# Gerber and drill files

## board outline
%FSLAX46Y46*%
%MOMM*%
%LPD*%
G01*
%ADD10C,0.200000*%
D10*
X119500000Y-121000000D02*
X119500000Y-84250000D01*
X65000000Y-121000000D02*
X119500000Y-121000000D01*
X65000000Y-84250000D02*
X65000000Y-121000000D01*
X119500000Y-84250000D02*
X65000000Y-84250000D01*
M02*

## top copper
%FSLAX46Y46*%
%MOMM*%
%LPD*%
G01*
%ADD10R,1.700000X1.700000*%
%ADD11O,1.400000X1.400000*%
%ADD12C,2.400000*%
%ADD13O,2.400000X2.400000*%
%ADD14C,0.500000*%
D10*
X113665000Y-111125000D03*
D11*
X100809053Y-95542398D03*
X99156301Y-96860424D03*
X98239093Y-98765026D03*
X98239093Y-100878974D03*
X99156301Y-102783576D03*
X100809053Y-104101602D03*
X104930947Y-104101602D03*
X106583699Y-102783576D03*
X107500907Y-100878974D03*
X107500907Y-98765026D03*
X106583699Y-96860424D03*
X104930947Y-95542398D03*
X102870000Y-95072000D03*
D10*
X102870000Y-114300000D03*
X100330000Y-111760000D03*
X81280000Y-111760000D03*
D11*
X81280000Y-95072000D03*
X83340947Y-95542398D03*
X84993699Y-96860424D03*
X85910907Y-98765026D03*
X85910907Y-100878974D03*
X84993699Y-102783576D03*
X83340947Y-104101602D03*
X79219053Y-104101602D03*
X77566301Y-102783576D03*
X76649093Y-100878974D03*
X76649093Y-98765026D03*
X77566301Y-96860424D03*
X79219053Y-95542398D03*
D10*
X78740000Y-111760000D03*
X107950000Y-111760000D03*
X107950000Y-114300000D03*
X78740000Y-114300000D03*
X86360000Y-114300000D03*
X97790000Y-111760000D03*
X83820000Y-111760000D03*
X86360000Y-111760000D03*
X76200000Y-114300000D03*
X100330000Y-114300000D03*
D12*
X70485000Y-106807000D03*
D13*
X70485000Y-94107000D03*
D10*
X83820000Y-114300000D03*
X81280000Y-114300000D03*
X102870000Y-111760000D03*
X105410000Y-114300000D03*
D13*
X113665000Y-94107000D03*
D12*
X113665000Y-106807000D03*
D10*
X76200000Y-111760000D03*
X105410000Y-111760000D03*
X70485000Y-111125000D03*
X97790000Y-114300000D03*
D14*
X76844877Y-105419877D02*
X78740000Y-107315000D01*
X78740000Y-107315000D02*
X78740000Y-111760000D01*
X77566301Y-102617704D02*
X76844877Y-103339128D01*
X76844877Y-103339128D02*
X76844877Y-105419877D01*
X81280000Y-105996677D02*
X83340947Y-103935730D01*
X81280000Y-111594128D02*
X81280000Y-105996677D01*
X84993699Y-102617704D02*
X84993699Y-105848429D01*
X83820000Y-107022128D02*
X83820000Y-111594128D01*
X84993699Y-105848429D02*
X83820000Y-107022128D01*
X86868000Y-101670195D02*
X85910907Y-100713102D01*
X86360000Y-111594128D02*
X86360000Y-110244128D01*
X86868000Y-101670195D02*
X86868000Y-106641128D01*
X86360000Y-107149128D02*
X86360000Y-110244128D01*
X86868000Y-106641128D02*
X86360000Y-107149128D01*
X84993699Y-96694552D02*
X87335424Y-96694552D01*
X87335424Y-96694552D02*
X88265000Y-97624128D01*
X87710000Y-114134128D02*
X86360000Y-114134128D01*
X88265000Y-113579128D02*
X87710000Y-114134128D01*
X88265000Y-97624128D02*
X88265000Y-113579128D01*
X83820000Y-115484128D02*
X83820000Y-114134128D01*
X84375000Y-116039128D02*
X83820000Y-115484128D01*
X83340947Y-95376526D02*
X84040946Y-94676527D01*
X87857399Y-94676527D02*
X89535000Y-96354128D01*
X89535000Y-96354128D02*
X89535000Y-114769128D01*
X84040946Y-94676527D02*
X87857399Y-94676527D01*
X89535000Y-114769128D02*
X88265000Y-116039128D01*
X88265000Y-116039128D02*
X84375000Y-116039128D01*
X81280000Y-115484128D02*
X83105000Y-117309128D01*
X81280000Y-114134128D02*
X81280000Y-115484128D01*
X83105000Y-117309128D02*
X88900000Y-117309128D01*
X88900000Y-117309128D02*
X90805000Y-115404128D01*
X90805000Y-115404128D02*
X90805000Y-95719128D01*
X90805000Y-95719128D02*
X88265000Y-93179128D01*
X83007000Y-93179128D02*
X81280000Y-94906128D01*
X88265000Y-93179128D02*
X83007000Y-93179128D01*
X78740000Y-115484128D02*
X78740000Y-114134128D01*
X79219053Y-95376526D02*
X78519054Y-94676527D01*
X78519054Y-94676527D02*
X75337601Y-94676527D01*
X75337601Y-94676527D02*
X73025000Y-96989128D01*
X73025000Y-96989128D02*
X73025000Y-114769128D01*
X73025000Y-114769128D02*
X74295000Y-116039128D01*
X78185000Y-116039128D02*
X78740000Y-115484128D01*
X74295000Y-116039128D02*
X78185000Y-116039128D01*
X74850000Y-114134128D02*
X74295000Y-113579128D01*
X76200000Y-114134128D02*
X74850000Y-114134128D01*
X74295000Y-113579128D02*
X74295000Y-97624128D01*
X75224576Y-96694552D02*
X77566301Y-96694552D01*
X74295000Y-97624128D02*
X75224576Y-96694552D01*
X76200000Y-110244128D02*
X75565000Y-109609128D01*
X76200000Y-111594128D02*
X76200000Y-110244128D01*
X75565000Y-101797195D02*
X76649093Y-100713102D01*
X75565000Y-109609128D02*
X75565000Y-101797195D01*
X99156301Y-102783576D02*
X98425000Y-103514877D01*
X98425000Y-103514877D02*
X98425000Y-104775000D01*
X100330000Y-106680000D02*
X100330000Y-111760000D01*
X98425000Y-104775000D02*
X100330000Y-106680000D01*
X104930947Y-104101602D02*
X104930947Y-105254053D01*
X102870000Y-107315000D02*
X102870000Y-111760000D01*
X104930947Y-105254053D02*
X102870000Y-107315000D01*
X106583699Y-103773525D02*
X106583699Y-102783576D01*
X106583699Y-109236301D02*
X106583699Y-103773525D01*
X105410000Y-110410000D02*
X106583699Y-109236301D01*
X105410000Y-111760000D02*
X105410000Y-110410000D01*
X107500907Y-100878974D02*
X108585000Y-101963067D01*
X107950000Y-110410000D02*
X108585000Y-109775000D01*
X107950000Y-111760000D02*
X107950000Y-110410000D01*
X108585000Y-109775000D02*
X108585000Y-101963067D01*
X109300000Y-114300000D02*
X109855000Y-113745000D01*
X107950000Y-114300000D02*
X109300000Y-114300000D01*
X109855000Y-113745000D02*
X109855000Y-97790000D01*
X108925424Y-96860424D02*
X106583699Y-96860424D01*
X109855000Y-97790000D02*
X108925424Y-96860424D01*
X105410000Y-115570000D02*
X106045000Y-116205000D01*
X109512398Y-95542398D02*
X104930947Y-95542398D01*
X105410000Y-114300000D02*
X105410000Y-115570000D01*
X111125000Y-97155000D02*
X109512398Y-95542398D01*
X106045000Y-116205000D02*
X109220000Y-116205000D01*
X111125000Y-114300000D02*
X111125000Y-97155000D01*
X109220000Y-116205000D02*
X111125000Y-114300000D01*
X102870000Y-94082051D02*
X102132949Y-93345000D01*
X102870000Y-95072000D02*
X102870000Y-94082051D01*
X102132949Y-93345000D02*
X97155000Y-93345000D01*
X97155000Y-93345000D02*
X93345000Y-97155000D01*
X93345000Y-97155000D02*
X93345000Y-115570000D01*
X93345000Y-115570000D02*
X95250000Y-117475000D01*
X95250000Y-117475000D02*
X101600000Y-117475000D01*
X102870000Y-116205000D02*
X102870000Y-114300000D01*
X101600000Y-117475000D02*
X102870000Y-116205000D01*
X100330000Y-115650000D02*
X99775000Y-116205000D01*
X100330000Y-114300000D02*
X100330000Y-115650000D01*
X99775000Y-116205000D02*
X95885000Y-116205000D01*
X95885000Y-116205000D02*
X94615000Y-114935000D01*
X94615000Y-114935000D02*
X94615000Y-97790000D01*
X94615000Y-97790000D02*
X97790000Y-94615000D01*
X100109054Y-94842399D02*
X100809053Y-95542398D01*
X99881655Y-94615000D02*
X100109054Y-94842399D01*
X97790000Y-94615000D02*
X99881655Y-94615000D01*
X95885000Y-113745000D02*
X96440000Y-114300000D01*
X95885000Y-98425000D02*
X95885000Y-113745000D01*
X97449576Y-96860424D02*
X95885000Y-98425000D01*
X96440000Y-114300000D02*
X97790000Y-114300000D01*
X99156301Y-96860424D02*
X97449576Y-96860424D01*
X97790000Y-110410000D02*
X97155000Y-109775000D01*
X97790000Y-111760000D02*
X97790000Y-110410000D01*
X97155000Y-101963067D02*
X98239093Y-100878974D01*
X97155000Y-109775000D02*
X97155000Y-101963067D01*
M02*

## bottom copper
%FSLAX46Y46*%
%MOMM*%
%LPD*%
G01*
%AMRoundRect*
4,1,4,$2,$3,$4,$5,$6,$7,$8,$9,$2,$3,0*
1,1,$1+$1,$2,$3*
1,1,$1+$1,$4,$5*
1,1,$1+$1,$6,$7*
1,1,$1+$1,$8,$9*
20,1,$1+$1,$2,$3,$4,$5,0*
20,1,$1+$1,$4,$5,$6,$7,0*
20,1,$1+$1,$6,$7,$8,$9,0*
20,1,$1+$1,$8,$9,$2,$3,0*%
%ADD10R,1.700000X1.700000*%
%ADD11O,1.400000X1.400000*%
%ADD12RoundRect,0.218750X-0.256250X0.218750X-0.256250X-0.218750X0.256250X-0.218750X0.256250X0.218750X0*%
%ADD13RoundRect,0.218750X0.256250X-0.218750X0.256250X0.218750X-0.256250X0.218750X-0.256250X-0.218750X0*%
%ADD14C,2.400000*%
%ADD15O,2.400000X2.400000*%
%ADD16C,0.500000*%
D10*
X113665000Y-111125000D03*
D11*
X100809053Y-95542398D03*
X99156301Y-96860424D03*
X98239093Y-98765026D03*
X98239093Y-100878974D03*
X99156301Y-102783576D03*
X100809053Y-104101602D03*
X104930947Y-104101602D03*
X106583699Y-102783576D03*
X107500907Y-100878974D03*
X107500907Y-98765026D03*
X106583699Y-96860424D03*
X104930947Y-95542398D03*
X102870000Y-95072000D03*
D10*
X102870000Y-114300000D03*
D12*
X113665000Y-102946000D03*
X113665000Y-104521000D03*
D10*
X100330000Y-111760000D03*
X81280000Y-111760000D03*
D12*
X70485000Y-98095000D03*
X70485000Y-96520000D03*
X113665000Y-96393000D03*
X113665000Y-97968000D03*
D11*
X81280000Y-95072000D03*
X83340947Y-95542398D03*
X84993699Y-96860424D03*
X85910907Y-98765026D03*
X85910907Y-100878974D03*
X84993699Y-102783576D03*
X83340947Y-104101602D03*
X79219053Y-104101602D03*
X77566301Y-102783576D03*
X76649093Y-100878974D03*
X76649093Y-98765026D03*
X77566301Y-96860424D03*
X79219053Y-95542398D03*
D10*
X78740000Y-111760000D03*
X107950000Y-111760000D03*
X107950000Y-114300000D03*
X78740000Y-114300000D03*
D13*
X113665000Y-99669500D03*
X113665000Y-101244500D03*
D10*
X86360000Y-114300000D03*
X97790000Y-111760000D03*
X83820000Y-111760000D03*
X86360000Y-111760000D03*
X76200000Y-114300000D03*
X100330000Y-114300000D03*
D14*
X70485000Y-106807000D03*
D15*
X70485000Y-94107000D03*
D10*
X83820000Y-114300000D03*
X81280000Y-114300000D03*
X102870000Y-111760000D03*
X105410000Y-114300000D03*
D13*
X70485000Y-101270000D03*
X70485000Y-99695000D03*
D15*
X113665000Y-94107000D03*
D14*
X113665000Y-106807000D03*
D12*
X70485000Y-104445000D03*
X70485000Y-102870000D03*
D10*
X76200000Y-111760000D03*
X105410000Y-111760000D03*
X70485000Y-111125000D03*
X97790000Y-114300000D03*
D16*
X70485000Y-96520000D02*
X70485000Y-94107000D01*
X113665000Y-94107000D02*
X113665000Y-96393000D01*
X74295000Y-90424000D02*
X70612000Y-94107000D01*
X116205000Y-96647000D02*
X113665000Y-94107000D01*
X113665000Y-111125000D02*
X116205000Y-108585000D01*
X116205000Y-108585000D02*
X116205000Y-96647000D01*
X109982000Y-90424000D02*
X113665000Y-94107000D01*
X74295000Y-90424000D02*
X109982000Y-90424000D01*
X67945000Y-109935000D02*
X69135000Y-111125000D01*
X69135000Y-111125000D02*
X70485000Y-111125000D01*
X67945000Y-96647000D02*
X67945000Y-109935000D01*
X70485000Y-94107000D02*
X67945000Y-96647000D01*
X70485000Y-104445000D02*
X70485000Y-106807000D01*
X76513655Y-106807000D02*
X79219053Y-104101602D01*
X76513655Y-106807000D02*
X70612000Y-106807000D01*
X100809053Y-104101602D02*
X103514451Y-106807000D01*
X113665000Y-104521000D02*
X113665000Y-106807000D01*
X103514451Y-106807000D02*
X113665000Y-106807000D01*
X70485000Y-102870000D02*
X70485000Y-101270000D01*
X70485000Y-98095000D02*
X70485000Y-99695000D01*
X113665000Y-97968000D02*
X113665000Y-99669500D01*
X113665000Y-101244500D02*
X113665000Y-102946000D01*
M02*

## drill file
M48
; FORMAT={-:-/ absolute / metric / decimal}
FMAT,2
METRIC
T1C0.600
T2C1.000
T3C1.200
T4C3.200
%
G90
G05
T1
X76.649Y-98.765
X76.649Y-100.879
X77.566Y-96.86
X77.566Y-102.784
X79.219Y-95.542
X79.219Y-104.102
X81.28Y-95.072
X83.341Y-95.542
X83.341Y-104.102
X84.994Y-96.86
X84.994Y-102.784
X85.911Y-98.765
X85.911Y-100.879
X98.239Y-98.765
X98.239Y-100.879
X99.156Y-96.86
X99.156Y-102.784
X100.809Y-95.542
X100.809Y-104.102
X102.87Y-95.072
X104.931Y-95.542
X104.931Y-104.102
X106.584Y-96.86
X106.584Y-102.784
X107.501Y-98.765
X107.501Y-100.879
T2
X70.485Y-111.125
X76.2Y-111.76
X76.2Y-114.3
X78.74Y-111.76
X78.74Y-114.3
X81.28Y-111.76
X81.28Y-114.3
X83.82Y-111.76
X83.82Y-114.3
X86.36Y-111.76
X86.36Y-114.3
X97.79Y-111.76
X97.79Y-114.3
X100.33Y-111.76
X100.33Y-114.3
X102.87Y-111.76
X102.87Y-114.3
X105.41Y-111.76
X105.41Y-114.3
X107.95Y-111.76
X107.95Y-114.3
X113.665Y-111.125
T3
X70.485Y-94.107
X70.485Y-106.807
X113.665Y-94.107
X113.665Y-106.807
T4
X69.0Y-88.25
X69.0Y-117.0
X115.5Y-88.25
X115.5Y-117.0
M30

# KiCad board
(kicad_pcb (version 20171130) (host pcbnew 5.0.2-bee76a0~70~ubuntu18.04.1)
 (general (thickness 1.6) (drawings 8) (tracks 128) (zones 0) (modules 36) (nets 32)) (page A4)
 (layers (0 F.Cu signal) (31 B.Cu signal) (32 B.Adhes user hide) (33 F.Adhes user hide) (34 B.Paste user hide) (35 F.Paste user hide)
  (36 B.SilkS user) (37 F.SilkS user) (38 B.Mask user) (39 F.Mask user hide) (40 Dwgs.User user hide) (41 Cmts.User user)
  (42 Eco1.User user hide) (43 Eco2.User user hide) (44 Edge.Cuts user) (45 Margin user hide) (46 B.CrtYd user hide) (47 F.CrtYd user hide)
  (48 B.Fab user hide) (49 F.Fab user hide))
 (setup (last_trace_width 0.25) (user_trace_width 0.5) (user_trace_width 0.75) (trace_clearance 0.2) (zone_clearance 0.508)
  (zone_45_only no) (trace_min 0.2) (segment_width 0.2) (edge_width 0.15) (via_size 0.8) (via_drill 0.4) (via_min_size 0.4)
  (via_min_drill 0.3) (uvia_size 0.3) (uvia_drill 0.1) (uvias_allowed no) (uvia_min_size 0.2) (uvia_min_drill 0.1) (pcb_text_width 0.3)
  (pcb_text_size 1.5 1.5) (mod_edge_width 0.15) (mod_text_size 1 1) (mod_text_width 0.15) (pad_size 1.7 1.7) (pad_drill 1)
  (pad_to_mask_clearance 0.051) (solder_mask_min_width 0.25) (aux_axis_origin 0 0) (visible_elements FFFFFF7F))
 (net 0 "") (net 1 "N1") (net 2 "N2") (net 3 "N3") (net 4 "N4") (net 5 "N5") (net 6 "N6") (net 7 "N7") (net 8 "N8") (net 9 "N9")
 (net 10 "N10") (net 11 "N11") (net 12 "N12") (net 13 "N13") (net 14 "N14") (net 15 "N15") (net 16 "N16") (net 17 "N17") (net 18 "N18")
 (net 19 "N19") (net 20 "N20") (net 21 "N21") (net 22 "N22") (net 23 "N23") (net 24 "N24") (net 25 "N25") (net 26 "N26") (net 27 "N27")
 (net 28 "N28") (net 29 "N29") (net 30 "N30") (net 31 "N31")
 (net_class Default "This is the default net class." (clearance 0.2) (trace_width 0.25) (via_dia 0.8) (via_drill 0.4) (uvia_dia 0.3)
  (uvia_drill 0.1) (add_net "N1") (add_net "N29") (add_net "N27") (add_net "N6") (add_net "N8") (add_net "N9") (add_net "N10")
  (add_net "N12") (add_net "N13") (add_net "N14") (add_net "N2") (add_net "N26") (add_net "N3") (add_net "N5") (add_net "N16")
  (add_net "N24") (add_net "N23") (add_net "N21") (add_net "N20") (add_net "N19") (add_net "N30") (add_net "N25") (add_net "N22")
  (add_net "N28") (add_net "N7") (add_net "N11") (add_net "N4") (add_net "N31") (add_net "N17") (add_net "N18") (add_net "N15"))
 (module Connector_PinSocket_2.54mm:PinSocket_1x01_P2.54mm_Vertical (layer F.Cu) (at 113.665 111.125)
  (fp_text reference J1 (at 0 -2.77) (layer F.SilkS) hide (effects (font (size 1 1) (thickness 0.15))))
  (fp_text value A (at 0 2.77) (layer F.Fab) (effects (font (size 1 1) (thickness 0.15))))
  (pad 1 thru_hole rect (at 0 0) (size 1.7 1.7) (drill 1) (layers *.Cu *.Mask) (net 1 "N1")))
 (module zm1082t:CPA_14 (layer F.Cu) (at 102.87 99.822)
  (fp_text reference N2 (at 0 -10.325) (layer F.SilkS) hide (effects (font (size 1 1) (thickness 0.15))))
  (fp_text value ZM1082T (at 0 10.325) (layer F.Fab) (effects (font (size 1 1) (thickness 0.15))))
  (pad 6 thru_hole oval (at -2.060947 -4.279602) (size 1.4 1.4) (drill 0.6) (layers *.Cu *.Mask) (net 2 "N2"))
  (pad 5 thru_hole oval (at -3.713699 -2.961576) (size 1.4 1.4) (drill 0.6) (layers *.Cu *.Mask) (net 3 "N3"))
  (pad 4 thru_hole oval (at -4.630907 -1.056974) (size 1.4 1.4) (drill 0.6) (layers *.Cu *.Mask) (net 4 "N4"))
  (pad 3 thru_hole oval (at -4.630907 1.056974) (size 1.4 1.4) (drill 0.6) (layers *.Cu *.Mask) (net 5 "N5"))
  (pad 2 thru_hole oval (at -3.713699 2.961576) (size 1.4 1.4) (drill 0.6) (layers *.Cu *.Mask) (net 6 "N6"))
  (pad 1 thru_hole oval (at -2.060947 4.279602) (size 1.4 1.4) (drill 0.6) (layers *.Cu *.Mask) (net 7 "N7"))
  (pad 13 thru_hole oval (at 2.060947 4.279602) (size 1.4 1.4) (drill 0.6) (layers *.Cu *.Mask) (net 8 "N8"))
  (pad 12 thru_hole oval (at 3.713699 2.961576) (size 1.4 1.4) (drill 0.6) (layers *.Cu *.Mask) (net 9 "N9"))
  (pad 11 thru_hole oval (at 4.630907 1.056974) (size 1.4 1.4) (drill 0.6) (layers *.Cu *.Mask) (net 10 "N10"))
  (pad 10 thru_hole oval (at 4.630907 -1.056974) (size 1.4 1.4) (drill 0.6) (layers *.Cu *.Mask) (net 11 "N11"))
  (pad 9 thru_hole oval (at 3.713699 -2.961576) (size 1.4 1.4) (drill 0.6) (layers *.Cu *.Mask) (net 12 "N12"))
  (pad 8 thru_hole oval (at 2.060947 -4.279602) (size 1.4 1.4) (drill 0.6) (layers *.Cu *.Mask) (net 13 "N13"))
  (pad 7 thru_hole oval (at 0 -4.75) (size 1.4 1.4) (drill 0.6) (layers *.Cu *.Mask) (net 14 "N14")))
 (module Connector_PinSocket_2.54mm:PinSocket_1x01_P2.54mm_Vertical (layer F.Cu) (at 102.87 114.3)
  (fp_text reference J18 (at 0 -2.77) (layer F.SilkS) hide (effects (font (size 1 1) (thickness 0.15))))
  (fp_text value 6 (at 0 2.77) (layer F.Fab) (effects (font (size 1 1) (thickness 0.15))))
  (pad 1 thru_hole rect (at 0 0) (size 1.7 1.7) (drill 1) (layers *.Cu *.Mask) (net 14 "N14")))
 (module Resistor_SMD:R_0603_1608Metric (layer B.Cu) (at 113.665 103.7335 270)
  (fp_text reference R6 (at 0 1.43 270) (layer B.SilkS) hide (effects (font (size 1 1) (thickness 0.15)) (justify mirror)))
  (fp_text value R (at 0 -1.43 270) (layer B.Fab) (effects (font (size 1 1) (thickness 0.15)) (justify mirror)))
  (pad 1 smd roundrect (at -0.7875 0 270) (size 0.875 0.95) (layers B.Cu B.Paste B.Mask) (roundrect_rratio 0.25) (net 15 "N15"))
  (pad 2 smd roundrect (at 0.7875 0 270) (size 0.875 0.95) (layers B.Cu B.Paste B.Mask) (roundrect_rratio 0.25) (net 7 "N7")))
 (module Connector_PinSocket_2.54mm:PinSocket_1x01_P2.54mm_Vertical (layer F.Cu) (at 100.33 111.76)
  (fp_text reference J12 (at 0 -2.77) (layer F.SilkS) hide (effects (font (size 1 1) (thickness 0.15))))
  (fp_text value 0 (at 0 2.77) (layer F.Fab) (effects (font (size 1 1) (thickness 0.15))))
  (pad 1 thru_hole rect (at 0 0) (size 1.7 1.7) (drill 1) (layers *.Cu *.Mask) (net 6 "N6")))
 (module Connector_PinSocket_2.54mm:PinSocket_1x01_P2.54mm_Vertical (layer F.Cu) (at 81.28 111.76)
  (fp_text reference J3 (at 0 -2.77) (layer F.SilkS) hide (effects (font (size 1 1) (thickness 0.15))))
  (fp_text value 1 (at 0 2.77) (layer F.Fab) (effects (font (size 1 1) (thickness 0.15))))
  (pad 1 thru_hole rect (at 0 0) (size 1.7 1.7) (drill 1) (layers *.Cu *.Mask) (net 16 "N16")))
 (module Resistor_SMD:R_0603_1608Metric (layer B.Cu) (at 70.485 97.3075 270)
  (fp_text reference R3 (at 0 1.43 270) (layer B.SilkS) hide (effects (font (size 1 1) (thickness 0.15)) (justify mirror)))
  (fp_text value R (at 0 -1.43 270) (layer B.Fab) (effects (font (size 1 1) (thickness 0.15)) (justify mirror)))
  (pad 2 smd roundrect (at 0.7875 0 270) (size 0.875 0.95) (layers B.Cu B.Paste B.Mask) (roundrect_rratio 0.25) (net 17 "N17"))
  (pad 1 smd roundrect (at -0.7875 0 270) (size 0.875 0.95) (layers B.Cu B.Paste B.Mask) (roundrect_rratio 0.25) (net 1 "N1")))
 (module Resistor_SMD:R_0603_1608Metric (layer B.Cu) (at 113.665 97.1805 270)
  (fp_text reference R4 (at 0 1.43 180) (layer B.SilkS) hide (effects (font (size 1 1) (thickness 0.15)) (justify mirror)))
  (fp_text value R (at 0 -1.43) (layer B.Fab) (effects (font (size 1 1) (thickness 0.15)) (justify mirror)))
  (pad 1 smd roundrect (at -0.7875 0 270) (size 0.875 0.95) (layers B.Cu B.Paste B.Mask) (roundrect_rratio 0.25) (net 1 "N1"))
  (pad 2 smd roundrect (at 0.7875 0 270) (size 0.875 0.95) (layers B.Cu B.Paste B.Mask) (roundrect_rratio 0.25) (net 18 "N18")))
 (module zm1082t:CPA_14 (layer F.Cu) (at 81.28 99.822)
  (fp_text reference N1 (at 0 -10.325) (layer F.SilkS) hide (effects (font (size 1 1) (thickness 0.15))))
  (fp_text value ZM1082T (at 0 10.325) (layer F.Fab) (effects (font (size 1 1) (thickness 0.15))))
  (pad 7 thru_hole oval (at 0 -4.75) (size 1.4 1.4) (drill 0.6) (layers *.Cu *.Mask) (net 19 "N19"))
  (pad 8 thru_hole oval (at 2.060947 -4.279602) (size 1.4 1.4) (drill 0.6) (layers *.Cu *.Mask) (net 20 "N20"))
  (pad 9 thru_hole oval (at 3.713699 -2.961576) (size 1.4 1.4) (drill 0.6) (layers *.Cu *.Mask) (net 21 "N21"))
  (pad 10 thru_hole oval (at 4.630907 -1.056974) (size 1.4 1.4) (drill 0.6) (layers *.Cu *.Mask) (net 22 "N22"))
  (pad 11 thru_hole oval (at 4.630907 1.056974) (size 1.4 1.4) (drill 0.6) (layers *.Cu *.Mask) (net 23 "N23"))
  (pad 12 thru_hole oval (at 3.713699 2.961576) (size 1.4 1.4) (drill 0.6) (layers *.Cu *.Mask) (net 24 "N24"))
  (pad 13 thru_hole oval (at 2.060947 4.279602) (size 1.4 1.4) (drill 0.6) (layers *.Cu *.Mask) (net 16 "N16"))
  (pad 1 thru_hole oval (at -2.060947 4.279602) (size 1.4 1.4) (drill 0.6) (layers *.Cu *.Mask) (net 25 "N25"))
  (pad 2 thru_hole oval (at -3.713699 2.961576) (size 1.4 1.4) (drill 0.6) (layers *.Cu *.Mask) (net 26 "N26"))
  (pad 3 thru_hole oval (at -4.630907 1.056974) (size 1.4 1.4) (drill 0.6) (layers *.Cu *.Mask) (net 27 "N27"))
  (pad 4 thru_hole oval (at -4.630907 -1.056974) (size 1.4 1.4) (drill 0.6) (layers *.Cu *.Mask) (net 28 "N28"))
  (pad 5 thru_hole oval (at -3.713699 -2.961576) (size 1.4 1.4) (drill 0.6) (layers *.Cu *.Mask) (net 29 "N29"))
  (pad 6 thru_hole oval (at -2.060947 -4.279602) (size 1.4 1.4) (drill 0.6) (layers *.Cu *.Mask) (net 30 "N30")))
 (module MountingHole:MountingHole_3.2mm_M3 (layer F.Cu) (at 69 88.25)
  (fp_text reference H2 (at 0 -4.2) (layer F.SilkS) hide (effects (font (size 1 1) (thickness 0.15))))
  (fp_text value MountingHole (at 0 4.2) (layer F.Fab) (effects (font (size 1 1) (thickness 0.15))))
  (pad 1 np_thru_hole circle (at 0 0) (size 3.2 3.2) (drill 3.2) (layers *.Cu *.Mask)))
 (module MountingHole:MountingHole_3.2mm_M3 (layer F.Cu) (at 115.5 117)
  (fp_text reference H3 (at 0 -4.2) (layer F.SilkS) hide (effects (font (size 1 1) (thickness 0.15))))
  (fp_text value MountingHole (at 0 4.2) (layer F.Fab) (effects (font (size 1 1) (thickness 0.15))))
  (pad 1 np_thru_hole circle (at 0 0) (size 3.2 3.2) (drill 3.2) (layers *.Cu *.Mask)))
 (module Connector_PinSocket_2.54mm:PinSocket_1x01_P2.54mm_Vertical (layer F.Cu) (at 78.74 113.03)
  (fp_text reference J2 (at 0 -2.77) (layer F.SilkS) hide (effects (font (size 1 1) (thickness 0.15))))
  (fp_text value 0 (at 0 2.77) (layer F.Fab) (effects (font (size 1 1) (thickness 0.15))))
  (pad 1 thru_hole rect (at 0 -1.27) (size 1.7 1.7) (drill 1) (layers *.Cu *.Mask) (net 26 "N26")))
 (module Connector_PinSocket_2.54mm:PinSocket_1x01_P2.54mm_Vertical (layer F.Cu) (at 107.95 111.76)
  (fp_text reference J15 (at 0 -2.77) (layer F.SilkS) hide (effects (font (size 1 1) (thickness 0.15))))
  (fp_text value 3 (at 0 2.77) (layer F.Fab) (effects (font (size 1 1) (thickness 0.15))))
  (pad 1 thru_hole rect (at 0 0) (size 1.7 1.7) (drill 1) (layers *.Cu *.Mask) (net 10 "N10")))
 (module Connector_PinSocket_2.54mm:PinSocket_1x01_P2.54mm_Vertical (layer F.Cu) (at 107.95 114.3)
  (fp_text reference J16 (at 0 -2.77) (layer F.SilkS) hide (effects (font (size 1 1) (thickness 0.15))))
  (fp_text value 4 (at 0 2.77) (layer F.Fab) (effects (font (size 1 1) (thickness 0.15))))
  (pad 1 thru_hole rect (at 0 0) (size 1.7 1.7) (drill 1) (layers *.Cu *.Mask) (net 12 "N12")))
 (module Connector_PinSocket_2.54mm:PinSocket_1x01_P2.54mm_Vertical (layer F.Cu) (at 78.74 114.3)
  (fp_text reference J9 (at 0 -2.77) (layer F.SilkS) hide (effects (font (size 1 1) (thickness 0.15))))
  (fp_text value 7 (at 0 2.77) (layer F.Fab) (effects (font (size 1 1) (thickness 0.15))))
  (pad 1 thru_hole rect (at 0 0) (size 1.7 1.7) (drill 1) (layers *.Cu *.Mask) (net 30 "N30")))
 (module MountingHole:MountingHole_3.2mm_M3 (layer F.Cu) (at 69 117)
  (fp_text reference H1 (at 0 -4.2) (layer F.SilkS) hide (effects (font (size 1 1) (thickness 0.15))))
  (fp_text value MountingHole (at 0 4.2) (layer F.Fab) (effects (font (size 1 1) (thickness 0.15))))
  (pad 1 np_thru_hole circle (at 0 0) (size 3.2 3.2) (drill 3.2) (layers *.Cu *.Mask)))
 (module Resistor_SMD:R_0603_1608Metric (layer B.Cu) (at 113.665 100.457 90)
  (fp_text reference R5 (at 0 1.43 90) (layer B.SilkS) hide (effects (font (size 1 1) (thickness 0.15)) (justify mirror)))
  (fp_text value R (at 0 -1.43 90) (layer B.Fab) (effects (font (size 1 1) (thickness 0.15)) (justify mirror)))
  (pad 2 smd roundrect (at 0.7875 0 90) (size 0.875 0.95) (layers B.Cu B.Paste B.Mask) (roundrect_rratio 0.25) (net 18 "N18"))
  (pad 1 smd roundrect (at -0.7875 0 90) (size 0.875 0.95) (layers B.Cu B.Paste B.Mask) (roundrect_rratio 0.25) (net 15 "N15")))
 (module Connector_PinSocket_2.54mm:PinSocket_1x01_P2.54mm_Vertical (layer F.Cu) (at 86.36 114.3)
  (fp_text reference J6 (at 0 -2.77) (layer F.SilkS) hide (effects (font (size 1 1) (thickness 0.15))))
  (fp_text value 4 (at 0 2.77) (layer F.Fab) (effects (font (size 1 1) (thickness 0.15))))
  (pad 1 thru_hole rect (at 0 0) (size 1.7 1.7) (drill 1) (layers *.Cu *.Mask) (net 21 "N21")))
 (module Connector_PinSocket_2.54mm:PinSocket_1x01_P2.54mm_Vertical (layer F.Cu) (at 97.79 111.76)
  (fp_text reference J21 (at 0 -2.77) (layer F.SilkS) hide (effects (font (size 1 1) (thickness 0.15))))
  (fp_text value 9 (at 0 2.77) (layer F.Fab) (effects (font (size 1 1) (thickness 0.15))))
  (pad 1 thru_hole rect (at 0 0) (size 1.7 1.7) (drill 1) (layers *.Cu *.Mask) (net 5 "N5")))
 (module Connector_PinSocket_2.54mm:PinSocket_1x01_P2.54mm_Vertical (layer F.Cu) (at 83.82 111.76)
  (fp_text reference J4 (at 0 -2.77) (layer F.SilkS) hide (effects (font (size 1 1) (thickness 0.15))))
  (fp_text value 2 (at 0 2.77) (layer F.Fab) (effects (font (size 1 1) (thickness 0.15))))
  (pad 1 thru_hole rect (at 0 0) (size 1.7 1.7) (drill 1) (layers *.Cu *.Mask) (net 24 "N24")))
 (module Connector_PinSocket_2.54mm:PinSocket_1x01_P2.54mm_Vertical (layer F.Cu) (at 86.36 111.76)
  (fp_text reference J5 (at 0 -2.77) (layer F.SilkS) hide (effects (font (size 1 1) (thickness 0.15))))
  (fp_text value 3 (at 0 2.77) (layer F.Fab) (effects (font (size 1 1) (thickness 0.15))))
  (pad 1 thru_hole rect (at 0 0) (size 1.7 1.7) (drill 1) (layers *.Cu *.Mask) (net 23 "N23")))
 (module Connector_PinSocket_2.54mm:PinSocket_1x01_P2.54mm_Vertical (layer F.Cu) (at 76.2 114.3)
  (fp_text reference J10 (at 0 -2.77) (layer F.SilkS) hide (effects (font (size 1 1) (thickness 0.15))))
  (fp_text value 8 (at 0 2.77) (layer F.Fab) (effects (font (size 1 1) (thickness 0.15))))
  (pad 1 thru_hole rect (at 0 0) (size 1.7 1.7) (drill 1) (layers *.Cu *.Mask) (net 29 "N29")))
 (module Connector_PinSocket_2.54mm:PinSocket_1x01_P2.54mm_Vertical (layer F.Cu) (at 100.33 114.3)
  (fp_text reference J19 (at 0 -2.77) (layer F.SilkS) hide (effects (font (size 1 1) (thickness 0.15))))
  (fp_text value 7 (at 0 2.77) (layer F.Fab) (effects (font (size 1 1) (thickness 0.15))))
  (pad 1 thru_hole rect (at 0 0) (size 1.7 1.7) (drill 1) (layers *.Cu *.Mask) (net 2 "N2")))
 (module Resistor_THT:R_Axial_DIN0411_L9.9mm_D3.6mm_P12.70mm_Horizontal (layer B.Cu) (at 70.485 106.807 90)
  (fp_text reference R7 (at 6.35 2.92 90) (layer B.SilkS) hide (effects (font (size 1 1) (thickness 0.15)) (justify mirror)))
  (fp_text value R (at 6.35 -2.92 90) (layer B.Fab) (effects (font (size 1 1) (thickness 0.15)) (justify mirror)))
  (pad 1 thru_hole circle (at 0 0 90) (size 2.4 2.4) (drill 1.2) (layers *.Cu *.Mask) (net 25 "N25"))
  (pad 2 thru_hole oval (at 12.7 0 90) (size 2.4 2.4) (drill 1.2) (layers *.Cu *.Mask) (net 1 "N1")))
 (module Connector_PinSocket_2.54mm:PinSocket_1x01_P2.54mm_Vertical (layer F.Cu) (at 83.82 114.3)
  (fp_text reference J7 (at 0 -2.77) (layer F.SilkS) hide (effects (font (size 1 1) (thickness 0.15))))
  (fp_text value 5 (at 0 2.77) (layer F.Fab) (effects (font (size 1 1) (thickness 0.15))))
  (pad 1 thru_hole rect (at 0 0) (size 1.7 1.7) (drill 1) (layers *.Cu *.Mask) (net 20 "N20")))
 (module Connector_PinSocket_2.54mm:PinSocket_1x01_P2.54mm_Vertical (layer F.Cu) (at 81.28 114.3)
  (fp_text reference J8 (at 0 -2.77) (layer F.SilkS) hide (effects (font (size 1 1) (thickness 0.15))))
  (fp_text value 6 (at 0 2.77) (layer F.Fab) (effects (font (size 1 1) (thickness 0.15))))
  (pad 1 thru_hole rect (at 0 0) (size 1.7 1.7) (drill 1) (layers *.Cu *.Mask) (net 19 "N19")))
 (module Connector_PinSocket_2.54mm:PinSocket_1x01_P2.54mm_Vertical (layer F.Cu) (at 102.87 111.76)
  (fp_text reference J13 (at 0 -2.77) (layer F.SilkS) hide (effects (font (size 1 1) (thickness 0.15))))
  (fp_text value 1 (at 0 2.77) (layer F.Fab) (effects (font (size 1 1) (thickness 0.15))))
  (pad 1 thru_hole rect (at 0 0) (size 1.7 1.7) (drill 1) (layers *.Cu *.Mask) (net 8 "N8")))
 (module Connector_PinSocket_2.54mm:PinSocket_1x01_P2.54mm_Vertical (layer F.Cu) (at 105.41 114.3)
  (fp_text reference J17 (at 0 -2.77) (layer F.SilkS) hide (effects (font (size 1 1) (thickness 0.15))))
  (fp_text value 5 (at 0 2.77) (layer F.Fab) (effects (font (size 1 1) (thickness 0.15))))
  (pad 1 thru_hole rect (at 0 0) (size 1.7 1.7) (drill 1) (layers *.Cu *.Mask) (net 13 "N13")))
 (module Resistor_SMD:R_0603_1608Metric (layer B.Cu) (at 70.485 100.4825 90)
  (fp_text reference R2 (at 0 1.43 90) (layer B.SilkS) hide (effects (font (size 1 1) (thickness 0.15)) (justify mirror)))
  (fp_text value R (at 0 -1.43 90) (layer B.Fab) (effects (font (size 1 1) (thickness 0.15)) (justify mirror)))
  (pad 1 smd roundrect (at -0.7875 0 90) (size 0.875 0.95) (layers B.Cu B.Paste B.Mask) (roundrect_rratio 0.25) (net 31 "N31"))
  (pad 2 smd roundrect (at 0.7875 0 90) (size 0.875 0.95) (layers B.Cu B.Paste B.Mask) (roundrect_rratio 0.25) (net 17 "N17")))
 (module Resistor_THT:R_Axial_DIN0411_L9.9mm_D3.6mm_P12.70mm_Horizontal (layer B.Cu) (at 113.665 106.807 90)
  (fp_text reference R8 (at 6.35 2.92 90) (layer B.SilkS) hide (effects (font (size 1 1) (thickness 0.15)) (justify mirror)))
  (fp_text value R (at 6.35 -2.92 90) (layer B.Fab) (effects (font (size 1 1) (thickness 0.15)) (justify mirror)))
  (pad 2 thru_hole oval (at 12.7 0 90) (size 2.4 2.4) (drill 1.2) (layers *.Cu *.Mask) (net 1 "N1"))
  (pad 1 thru_hole circle (at 0 0 90) (size 2.4 2.4) (drill 1.2) (layers *.Cu *.Mask) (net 7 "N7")))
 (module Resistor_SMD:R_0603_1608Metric (layer B.Cu) (at 70.485 103.6575 270)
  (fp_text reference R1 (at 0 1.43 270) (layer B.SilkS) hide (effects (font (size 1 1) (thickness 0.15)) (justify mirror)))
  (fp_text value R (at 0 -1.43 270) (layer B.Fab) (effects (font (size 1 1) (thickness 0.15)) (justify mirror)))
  (pad 2 smd roundrect (at 0.7875 0 270) (size 0.875 0.95) (layers B.Cu B.Paste B.Mask) (roundrect_rratio 0.25) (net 25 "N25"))
  (pad 1 smd roundrect (at -0.7875 0 270) (size 0.875 0.95) (layers B.Cu B.Paste B.Mask) (roundrect_rratio 0.25) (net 31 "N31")))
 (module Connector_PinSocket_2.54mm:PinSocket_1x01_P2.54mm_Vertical (layer F.Cu) (at 76.2 111.76)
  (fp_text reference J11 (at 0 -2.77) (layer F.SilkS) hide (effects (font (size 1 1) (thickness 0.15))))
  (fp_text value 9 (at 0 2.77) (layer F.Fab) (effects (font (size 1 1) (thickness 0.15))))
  (pad 1 thru_hole rect (at 0 0) (size 1.7 1.7) (drill 1) (layers *.Cu *.Mask) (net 27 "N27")))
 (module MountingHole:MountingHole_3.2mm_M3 (layer F.Cu) (at 115.5 88.25)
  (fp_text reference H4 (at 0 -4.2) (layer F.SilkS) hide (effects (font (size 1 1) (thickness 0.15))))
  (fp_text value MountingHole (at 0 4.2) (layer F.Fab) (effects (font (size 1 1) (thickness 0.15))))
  (pad 1 np_thru_hole circle (at 0 0) (size 3.2 3.2) (drill 3.2) (layers *.Cu *.Mask)))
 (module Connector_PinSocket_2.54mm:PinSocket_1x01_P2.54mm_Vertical (layer F.Cu) (at 105.41 111.76)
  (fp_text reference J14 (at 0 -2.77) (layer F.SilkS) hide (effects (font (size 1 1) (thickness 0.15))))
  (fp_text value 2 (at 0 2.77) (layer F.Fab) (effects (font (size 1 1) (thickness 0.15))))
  (pad 1 thru_hole rect (at 0 0) (size 1.7 1.7) (drill 1) (layers *.Cu *.Mask) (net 9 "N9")))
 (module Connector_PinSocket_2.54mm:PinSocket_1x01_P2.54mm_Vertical (layer F.Cu) (at 70.485 111.125)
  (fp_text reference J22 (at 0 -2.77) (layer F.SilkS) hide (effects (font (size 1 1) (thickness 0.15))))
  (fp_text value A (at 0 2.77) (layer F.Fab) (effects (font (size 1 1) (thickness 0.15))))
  (pad 1 thru_hole rect (at 0 0) (size 1.7 1.7) (drill 1) (layers *.Cu *.Mask) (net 1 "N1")))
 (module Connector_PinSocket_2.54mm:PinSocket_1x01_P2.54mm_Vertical (layer F.Cu) (at 97.79 114.3)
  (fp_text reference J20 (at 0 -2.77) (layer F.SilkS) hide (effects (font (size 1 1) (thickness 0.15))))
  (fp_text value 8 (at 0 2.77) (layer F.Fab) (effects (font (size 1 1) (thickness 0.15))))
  (pad 1 thru_hole rect (at 0 0) (size 1.7 1.7) (drill 1) (layers *.Cu *.Mask) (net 3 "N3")))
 (gr_line (start 119.5 121) (end 119.5 84.25) (layer Edge.Cuts) (width 0.2))
 (gr_line (start 65 121) (end 119.5 121) (layer Edge.Cuts) (width 0.2))
 (gr_line (start 65 84.25) (end 65 121) (layer Edge.Cuts) (width 0.2))
 (gr_line (start 119.5 84.25) (end 65 84.25) (layer Edge.Cuts) (width 0.2))
 (segment (start 70.485 96.52) (end 70.485 94.107) (width 0.5) (layer B.Cu) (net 1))
 (segment (start 113.665 94.107) (end 113.665 96.393) (width 0.5) (layer B.Cu) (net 1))
 (segment (start 74.295 90.424) (end 70.612 94.107) (width 0.5) (layer B.Cu) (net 1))
 (segment (start 116.205 96.647) (end 113.665 94.107) (width 0.5) (layer B.Cu) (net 1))
 (segment (start 113.665 111.125) (end 116.205 108.585) (width 0.5) (layer B.Cu) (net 1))
 (segment (start 116.205 108.585) (end 116.205 96.647) (width 0.5) (layer B.Cu) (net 1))
 (segment (start 109.982 90.424) (end 113.665 94.107) (width 0.5) (layer B.Cu) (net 1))
 (segment (start 74.295 90.424) (end 109.982 90.424) (width 0.5) (layer B.Cu) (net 1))
 (segment (start 67.945 109.935) (end 69.135 111.125) (width 0.5) (layer B.Cu) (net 1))
 (segment (start 69.135 111.125) (end 70.485 111.125) (width 0.5) (layer B.Cu) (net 1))
 (segment (start 67.945 96.647) (end 67.945 109.935) (width 0.5) (layer B.Cu) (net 1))
 (segment (start 70.485 94.107) (end 67.945 96.647) (width 0.5) (layer B.Cu) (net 1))
 (segment (start 76.844877 105.419877) (end 78.74 107.315) (width 0.5) (layer F.Cu) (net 26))
 (segment (start 78.74 107.315) (end 78.74 111.76) (width 0.5) (layer F.Cu) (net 26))
 (segment (start 77.566301 102.617704) (end 76.844877 103.339128) (width 0.5) (layer F.Cu) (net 26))
 (segment (start 76.844877 103.339128) (end 76.844877 105.419877) (width 0.5) (layer F.Cu) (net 26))
 (segment (start 81.28 105.996677) (end 83.340947 103.93573) (width 0.5) (layer F.Cu) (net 16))
 (segment (start 81.28 111.594128) (end 81.28 105.996677) (width 0.5) (layer F.Cu) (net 16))
 (segment (start 84.993699 102.617704) (end 84.993699 105.848429) (width 0.5) (layer F.Cu) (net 24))
 (segment (start 83.82 107.022128) (end 83.82 111.594128) (width 0.5) (layer F.Cu) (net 24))
 (segment (start 84.993699 105.848429) (end 83.82 107.022128) (width 0.5) (layer F.Cu) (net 24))
 (segment (start 86.868 101.670195) (end 85.910907 100.713102) (width 0.5) (layer F.Cu) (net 23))
 (segment (start 86.36 111.594128) (end 86.36 110.244128) (width 0.5) (layer F.Cu) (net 23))
 (segment (start 86.868 101.670195) (end 86.868 106.641128) (width 0.5) (layer F.Cu) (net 23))
 (segment (start 86.36 107.149128) (end 86.36 110.244128) (width 0.5) (layer F.Cu) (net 23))
 (segment (start 86.868 106.641128) (end 86.36 107.149128) (width 0.5) (layer F.Cu) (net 23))
 (segment (start 84.993699 96.694552) (end 87.335424 96.694552) (width 0.5) (layer F.Cu) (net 21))
 (segment (start 87.335424 96.694552) (end 88.265 97.624128) (width 0.5) (layer F.Cu) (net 21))
 (segment (start 87.71 114.134128) (end 86.36 114.134128) (width 0.5) (layer F.Cu) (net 21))
 (segment (start 88.265 113.579128) (end 87.71 114.134128) (width 0.5) (layer F.Cu) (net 21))
 (segment (start 88.265 97.624128) (end 88.265 113.579128) (width 0.5) (layer F.Cu) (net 21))
 (segment (start 83.82 115.484128) (end 83.82 114.134128) (width 0.5) (layer F.Cu) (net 20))
 (segment (start 84.375 116.039128) (end 83.82 115.484128) (width 0.5) (layer F.Cu) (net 20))
 (segment (start 83.340947 95.376526) (end 84.040946 94.676527) (width 0.5) (layer F.Cu) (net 20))
 (segment (start 87.857399 94.676527) (end 89.535 96.354128) (width 0.5) (layer F.Cu) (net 20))
 (segment (start 89.535 96.354128) (end 89.535 114.769128) (width 0.5) (layer F.Cu) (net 20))
 (segment (start 84.040946 94.676527) (end 87.857399 94.676527) (width 0.5) (layer F.Cu) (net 20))
 (segment (start 89.535 114.769128) (end 88.265 116.039128) (width 0.5) (layer F.Cu) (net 20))
 (segment (start 88.265 116.039128) (end 84.375 116.039128) (width 0.5) (layer F.Cu) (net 20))
 (segment (start 81.28 115.484128) (end 83.105 117.309128) (width 0.5) (layer F.Cu) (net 19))
 (segment (start 81.28 114.134128) (end 81.28 115.484128) (width 0.5) (layer F.Cu) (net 19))
 (segment (start 83.105 117.309128) (end 88.9 117.309128) (width 0.5) (layer F.Cu) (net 19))
 (segment (start 88.9 117.309128) (end 90.805 115.404128) (width 0.5) (layer F.Cu) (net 19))
 (segment (start 90.805 115.404128) (end 90.805 95.719128) (width 0.5) (layer F.Cu) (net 19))
 (segment (start 90.805 95.719128) (end 88.265 93.179128) (width 0.5) (layer F.Cu) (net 19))
 (segment (start 83.007 93.179128) (end 81.28 94.906128) (width 0.5) (layer F.Cu) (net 19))
 (segment (start 88.265 93.179128) (end 83.007 93.179128) (width 0.5) (layer F.Cu) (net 19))
 (segment (start 78.74 115.484128) (end 78.74 114.134128) (width 0.5) (layer F.Cu) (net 30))
 (segment (start 79.219053 95.376526) (end 78.519054 94.676527) (width 0.5) (layer F.Cu) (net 30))
 (segment (start 78.519054 94.676527) (end 75.337601 94.676527) (width 0.5) (layer F.Cu) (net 30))
 (segment (start 75.337601 94.676527) (end 73.025 96.989128) (width 0.5) (layer F.Cu) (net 30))
 (segment (start 73.025 96.989128) (end 73.025 114.769128) (width 0.5) (layer F.Cu) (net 30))
 (segment (start 73.025 114.769128) (end 74.295 116.039128) (width 0.5) (layer F.Cu) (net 30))
 (segment (start 78.185 116.039128) (end 78.74 115.484128) (width 0.5) (layer F.Cu) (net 30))
 (segment (start 74.295 116.039128) (end 78.185 116.039128) (width 0.5) (layer F.Cu) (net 30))
 (segment (start 74.85 114.134128) (end 74.295 113.579128) (width 0.5) (layer F.Cu) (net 29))
 (segment (start 76.2 114.134128) (end 74.85 114.134128) (width 0.5) (layer F.Cu) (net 29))
 (segment (start 74.295 113.579128) (end 74.295 97.624128) (width 0.5) (layer F.Cu) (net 29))
 (segment (start 75.224576 96.694552) (end 77.566301 96.694552) (width 0.5) (layer F.Cu) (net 29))
 (segment (start 74.295 97.624128) (end 75.224576 96.694552) (width 0.5) (layer F.Cu) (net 29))
 (segment (start 76.2 110.244128) (end 75.565 109.609128) (width 0.5) (layer F.Cu) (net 27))
 (segment (start 76.2 111.594128) (end 76.2 110.244128) (width 0.5) (layer F.Cu) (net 27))
 (segment (start 75.565 101.797195) (end 76.649093 100.713102) (width 0.5) (layer F.Cu) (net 27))
 (segment (start 75.565 109.609128) (end 75.565 101.797195) (width 0.5) (layer F.Cu) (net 27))
 (segment (start 99.156301 102.783576) (end 98.425 103.514877) (width 0.5) (layer F.Cu) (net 6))
 (segment (start 98.425 103.514877) (end 98.425 104.775) (width 0.5) (layer F.Cu) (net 6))
 (segment (start 100.33 106.68) (end 100.33 111.76) (width 0.5) (layer F.Cu) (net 6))
 (segment (start 98.425 104.775) (end 100.33 106.68) (width 0.5) (layer F.Cu) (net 6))
 (segment (start 104.930947 104.101602) (end 104.930947 105.254053) (width 0.5) (layer F.Cu) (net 8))
 (segment (start 102.87 107.315) (end 102.87 111.76) (width 0.5) (layer F.Cu) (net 8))
 (segment (start 104.930947 105.254053) (end 102.87 107.315) (width 0.5) (layer F.Cu) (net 8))
 (segment (start 106.583699 103.773525) (end 106.583699 102.783576) (width 0.5) (layer F.Cu) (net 9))
 (segment (start 106.583699 109.236301) (end 106.583699 103.773525) (width 0.5) (layer F.Cu) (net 9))
 (segment (start 105.41 110.41) (end 106.583699 109.236301) (width 0.5) (layer F.Cu) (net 9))
 (segment (start 105.41 111.76) (end 105.41 110.41) (width 0.5) (layer F.Cu) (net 9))
 (segment (start 107.500907 100.878974) (end 108.585 101.963067) (width 0.5) (layer F.Cu) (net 10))
 (segment (start 107.95 110.41) (end 108.585 109.775) (width 0.5) (layer F.Cu) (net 10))
 (segment (start 107.95 111.76) (end 107.95 110.41) (width 0.5) (layer F.Cu) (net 10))
 (segment (start 108.585 109.775) (end 108.585 101.963067) (width 0.5) (layer F.Cu) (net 10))
 (segment (start 109.3 114.3) (end 109.855 113.745) (width 0.5) (layer F.Cu) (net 12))
 (segment (start 107.95 114.3) (end 109.3 114.3) (width 0.5) (layer F.Cu) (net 12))
 (segment (start 109.855 113.745) (end 109.855 97.79) (width 0.5) (layer F.Cu) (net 12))
 (segment (start 108.925424 96.860424) (end 106.583699 96.860424) (width 0.5) (layer F.Cu) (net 12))
 (segment (start 109.855 97.79) (end 108.925424 96.860424) (width 0.5) (layer F.Cu) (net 12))
 (segment (start 105.41 115.57) (end 106.045 116.205) (width 0.5) (layer F.Cu) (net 13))
 (segment (start 109.512398 95.542398) (end 104.930947 95.542398) (width 0.5) (layer F.Cu) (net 13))
 (segment (start 105.41 114.3) (end 105.41 115.57) (width 0.5) (layer F.Cu) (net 13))
 (segment (start 111.125 97.155) (end 109.512398 95.542398) (width 0.5) (layer F.Cu) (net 13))
 (segment (start 106.045 116.205) (end 109.22 116.205) (width 0.5) (layer F.Cu) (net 13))
 (segment (start 111.125 114.3) (end 111.125 97.155) (width 0.5) (layer F.Cu) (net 13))
 (segment (start 109.22 116.205) (end 111.125 114.3) (width 0.5) (layer F.Cu) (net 13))
 (segment (start 102.87 94.082051) (end 102.132949 93.345) (width 0.5) (layer F.Cu) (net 14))
 (segment (start 102.87 95.072) (end 102.87 94.082051) (width 0.5) (layer F.Cu) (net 14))
 (segment (start 102.132949 93.345) (end 97.155 93.345) (width 0.5) (layer F.Cu) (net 14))
 (segment (start 97.155 93.345) (end 93.345 97.155) (width 0.5) (layer F.Cu) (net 14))
 (segment (start 93.345 97.155) (end 93.345 115.57) (width 0.5) (layer F.Cu) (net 14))
 (segment (start 93.345 115.57) (end 95.25 117.475) (width 0.5) (layer F.Cu) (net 14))
 (segment (start 95.25 117.475) (end 101.6 117.475) (width 0.5) (layer F.Cu) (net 14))
 (segment (start 102.87 116.205) (end 102.87 114.3) (width 0.5) (layer F.Cu) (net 14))
 (segment (start 101.6 117.475) (end 102.87 116.205) (width 0.5) (layer F.Cu) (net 14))
 (segment (start 100.33 115.65) (end 99.775 116.205) (width 0.5) (layer F.Cu) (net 2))
 (segment (start 100.33 114.3) (end 100.33 115.65) (width 0.5) (layer F.Cu) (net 2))
 (segment (start 99.775 116.205) (end 95.885 116.205) (width 0.5) (layer F.Cu) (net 2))
 (segment (start 95.885 116.205) (end 94.615 114.935) (width 0.5) (layer F.Cu) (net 2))
 (segment (start 94.615 114.935) (end 94.615 97.79) (width 0.5) (layer F.Cu) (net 2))
 (segment (start 94.615 97.79) (end 97.79 94.615) (width 0.5) (layer F.Cu) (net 2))
 (segment (start 100.109054 94.842399) (end 100.809053 95.542398) (width 0.5) (layer F.Cu) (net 2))
 (segment (start 99.881655 94.615) (end 100.109054 94.842399) (width 0.5) (layer F.Cu) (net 2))
 (segment (start 97.79 94.615) (end 99.881655 94.615) (width 0.5) (layer F.Cu) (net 2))
 (segment (start 95.885 113.745) (end 96.44 114.3) (width 0.5) (layer F.Cu) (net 3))
 (segment (start 95.885 98.425) (end 95.885 113.745) (width 0.5) (layer F.Cu) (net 3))
 (segment (start 97.449576 96.860424) (end 95.885 98.425) (width 0.5) (layer F.Cu) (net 3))
 (segment (start 96.44 114.3) (end 97.79 114.3) (width 0.5) (layer F.Cu) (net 3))
 (segment (start 99.156301 96.860424) (end 97.449576 96.860424) (width 0.5) (layer F.Cu) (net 3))
 (segment (start 97.79 110.41) (end 97.155 109.775) (width 0.5) (layer F.Cu) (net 5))
 (segment (start 97.79 111.76) (end 97.79 110.41) (width 0.5) (layer F.Cu) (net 5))
 (segment (start 97.155 101.963067) (end 98.239093 100.878974) (width 0.5) (layer F.Cu) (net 5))
 (segment (start 97.155 109.775) (end 97.155 101.963067) (width 0.5) (layer F.Cu) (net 5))
 (segment (start 70.485 104.445) (end 70.485 106.807) (width 0.5) (layer B.Cu) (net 25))
 (segment (start 76.513655 106.807) (end 79.219053 104.101602) (width 0.5) (layer B.Cu) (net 25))
 (segment (start 76.513655 106.807) (end 70.612 106.807) (width 0.5) (layer B.Cu) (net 25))
 (segment (start 100.809053 104.101602) (end 103.514451 106.807) (width 0.5) (layer B.Cu) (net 7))
 (segment (start 113.665 104.521) (end 113.665 106.807) (width 0.5) (layer B.Cu) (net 7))
 (segment (start 103.514451 106.807) (end 113.665 106.807) (width 0.5) (layer B.Cu) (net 7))
 (segment (start 70.485 102.87) (end 70.485 101.27) (width 0.5) (layer B.Cu) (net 31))
 (segment (start 70.485 98.095) (end 70.485 99.695) (width 0.5) (layer B.Cu) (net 17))
 (segment (start 113.665 97.968) (end 113.665 99.6695) (width 0.5) (layer B.Cu) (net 18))
 (segment (start 113.665 101.2445) (end 113.665 102.946) (width 0.5) (layer B.Cu) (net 15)))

